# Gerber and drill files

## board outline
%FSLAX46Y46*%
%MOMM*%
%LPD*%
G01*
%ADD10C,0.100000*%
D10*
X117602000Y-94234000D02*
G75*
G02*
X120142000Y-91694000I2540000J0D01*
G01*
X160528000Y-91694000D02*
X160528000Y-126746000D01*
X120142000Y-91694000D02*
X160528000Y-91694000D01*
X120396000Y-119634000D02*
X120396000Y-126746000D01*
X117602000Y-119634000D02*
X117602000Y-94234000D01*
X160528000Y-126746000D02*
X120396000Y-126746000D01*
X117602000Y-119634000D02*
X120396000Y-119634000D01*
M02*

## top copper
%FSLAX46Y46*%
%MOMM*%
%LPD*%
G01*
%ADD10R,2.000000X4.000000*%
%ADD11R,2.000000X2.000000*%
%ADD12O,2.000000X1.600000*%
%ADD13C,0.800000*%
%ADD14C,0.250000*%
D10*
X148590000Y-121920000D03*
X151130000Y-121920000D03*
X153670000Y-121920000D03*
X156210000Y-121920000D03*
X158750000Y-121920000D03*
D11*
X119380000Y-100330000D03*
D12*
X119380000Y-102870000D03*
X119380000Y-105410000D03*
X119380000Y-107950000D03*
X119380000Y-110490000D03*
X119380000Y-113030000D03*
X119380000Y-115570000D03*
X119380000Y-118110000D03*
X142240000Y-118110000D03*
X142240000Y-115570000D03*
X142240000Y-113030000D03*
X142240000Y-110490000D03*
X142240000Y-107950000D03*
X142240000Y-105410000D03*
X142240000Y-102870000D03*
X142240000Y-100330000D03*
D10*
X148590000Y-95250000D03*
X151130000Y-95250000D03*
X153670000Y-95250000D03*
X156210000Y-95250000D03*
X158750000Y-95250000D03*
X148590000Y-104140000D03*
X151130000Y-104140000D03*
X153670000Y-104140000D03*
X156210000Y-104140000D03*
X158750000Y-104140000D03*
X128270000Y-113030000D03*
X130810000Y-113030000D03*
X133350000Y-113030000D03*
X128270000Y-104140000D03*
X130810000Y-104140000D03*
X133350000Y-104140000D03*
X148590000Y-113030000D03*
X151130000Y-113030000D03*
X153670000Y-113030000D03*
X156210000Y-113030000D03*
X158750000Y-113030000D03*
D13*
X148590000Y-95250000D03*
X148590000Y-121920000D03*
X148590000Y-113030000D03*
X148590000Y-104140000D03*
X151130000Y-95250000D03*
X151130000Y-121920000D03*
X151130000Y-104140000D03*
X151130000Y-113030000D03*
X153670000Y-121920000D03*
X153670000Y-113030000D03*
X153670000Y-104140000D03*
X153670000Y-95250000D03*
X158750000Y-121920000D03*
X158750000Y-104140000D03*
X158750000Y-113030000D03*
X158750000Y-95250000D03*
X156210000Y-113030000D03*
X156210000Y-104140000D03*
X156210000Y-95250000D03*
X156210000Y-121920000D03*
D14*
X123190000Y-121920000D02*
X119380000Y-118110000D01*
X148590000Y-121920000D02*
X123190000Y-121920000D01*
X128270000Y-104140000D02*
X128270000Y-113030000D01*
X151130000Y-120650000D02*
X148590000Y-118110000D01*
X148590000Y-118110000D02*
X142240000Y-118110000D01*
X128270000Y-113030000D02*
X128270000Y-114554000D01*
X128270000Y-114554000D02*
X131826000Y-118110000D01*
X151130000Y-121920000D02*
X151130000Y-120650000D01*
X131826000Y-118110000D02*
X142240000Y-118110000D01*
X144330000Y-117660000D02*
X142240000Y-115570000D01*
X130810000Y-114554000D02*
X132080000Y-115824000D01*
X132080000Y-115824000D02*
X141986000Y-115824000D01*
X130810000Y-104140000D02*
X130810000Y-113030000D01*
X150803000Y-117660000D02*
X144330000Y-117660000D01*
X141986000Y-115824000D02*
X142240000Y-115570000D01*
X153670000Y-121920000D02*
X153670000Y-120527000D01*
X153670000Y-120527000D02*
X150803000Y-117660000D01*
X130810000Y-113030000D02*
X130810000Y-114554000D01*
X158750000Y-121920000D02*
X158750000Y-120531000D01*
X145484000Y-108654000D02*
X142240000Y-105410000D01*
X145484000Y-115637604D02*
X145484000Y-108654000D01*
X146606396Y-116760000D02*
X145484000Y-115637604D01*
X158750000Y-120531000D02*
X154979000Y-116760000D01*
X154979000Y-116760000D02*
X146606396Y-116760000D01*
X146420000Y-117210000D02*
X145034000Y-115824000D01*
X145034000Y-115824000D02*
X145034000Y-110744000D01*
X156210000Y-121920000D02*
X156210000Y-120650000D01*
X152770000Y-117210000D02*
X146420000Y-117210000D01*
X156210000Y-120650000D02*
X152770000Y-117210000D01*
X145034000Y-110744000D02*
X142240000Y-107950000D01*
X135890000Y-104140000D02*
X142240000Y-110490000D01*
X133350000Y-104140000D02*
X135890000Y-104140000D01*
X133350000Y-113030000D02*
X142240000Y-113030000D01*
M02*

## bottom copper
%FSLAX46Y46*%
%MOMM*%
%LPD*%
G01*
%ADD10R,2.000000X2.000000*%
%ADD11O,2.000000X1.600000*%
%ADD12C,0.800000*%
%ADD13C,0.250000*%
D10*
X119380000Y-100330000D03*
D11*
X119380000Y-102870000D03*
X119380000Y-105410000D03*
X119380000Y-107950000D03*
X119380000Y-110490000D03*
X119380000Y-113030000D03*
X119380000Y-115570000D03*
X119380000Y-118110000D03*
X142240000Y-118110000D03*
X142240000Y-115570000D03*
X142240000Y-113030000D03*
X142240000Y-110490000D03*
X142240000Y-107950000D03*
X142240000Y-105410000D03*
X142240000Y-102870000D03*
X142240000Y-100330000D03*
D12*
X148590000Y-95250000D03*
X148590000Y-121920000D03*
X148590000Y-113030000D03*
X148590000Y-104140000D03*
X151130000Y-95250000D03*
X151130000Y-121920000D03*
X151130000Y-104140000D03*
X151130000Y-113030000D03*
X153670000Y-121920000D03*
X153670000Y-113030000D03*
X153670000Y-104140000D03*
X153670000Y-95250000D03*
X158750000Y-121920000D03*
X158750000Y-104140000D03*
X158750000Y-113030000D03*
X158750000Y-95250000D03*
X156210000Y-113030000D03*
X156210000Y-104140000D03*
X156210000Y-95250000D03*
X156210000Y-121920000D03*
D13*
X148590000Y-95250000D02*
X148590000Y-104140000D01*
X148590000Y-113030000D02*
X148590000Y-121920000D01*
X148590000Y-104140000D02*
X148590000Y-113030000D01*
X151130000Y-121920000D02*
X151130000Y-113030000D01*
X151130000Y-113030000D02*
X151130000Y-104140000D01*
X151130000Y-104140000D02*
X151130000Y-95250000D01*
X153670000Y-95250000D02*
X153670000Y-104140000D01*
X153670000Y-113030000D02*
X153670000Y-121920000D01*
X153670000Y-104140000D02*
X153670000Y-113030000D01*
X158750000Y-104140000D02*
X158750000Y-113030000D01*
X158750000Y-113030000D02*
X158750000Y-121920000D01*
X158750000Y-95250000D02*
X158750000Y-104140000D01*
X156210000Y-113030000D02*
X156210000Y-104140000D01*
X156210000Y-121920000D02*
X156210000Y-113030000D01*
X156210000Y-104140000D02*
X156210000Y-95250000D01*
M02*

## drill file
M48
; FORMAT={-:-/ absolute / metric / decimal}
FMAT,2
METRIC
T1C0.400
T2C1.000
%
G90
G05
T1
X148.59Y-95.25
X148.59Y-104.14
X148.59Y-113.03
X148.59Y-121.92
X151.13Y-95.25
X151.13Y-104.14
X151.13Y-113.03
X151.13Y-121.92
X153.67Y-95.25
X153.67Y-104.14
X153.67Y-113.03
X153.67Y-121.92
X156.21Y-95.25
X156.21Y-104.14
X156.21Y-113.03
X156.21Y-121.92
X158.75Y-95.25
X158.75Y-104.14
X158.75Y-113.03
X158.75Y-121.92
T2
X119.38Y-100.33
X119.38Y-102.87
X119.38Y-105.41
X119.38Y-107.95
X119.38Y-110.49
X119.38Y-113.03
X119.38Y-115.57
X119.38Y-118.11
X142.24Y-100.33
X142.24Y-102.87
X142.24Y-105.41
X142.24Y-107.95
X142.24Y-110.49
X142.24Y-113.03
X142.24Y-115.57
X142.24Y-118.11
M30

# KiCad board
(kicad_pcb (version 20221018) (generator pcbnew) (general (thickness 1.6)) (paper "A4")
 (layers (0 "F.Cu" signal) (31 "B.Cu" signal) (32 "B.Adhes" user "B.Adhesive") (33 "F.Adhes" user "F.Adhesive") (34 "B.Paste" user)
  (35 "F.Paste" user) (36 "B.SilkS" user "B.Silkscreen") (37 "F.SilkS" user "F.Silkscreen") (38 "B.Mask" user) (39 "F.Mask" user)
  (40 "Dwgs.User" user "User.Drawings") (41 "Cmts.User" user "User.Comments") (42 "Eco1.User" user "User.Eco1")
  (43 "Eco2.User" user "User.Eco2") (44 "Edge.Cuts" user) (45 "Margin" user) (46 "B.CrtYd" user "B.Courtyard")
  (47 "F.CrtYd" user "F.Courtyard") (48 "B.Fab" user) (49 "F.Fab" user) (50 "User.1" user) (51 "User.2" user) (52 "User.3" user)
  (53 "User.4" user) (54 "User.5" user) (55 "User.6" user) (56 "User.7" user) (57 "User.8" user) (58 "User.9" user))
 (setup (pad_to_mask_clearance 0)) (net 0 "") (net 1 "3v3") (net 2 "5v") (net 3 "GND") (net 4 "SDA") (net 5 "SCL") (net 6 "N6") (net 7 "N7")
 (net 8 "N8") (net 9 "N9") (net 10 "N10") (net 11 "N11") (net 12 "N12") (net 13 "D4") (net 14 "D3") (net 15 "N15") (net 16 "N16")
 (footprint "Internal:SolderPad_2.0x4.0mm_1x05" (layer "F.Cu") (at 153.67 124.46)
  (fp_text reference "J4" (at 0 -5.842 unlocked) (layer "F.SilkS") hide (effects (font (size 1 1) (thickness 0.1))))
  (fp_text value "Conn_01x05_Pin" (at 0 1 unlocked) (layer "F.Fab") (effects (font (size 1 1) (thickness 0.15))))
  (pad "1" smd rect (at -5.08 -2.54) (size 2 4) (layers "F.Cu" "F.Paste" "F.Mask") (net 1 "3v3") (thermal_bridge_angle 45))
  (pad "2" smd rect (at -2.54 -2.54) (size 2 4) (layers "F.Cu" "F.Paste" "F.Mask") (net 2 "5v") (thermal_bridge_angle 45))
  (pad "3" smd rect (at 0 -2.54) (size 2 4) (layers "F.Cu" "F.Paste" "F.Mask") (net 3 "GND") (thermal_bridge_angle 45))
  (pad "4" smd rect (at 2.54 -2.54) (size 2 4) (layers "F.Cu" "F.Paste" "F.Mask") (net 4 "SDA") (thermal_bridge_angle 45))
  (pad "5" smd rect (at 5.08 -2.54) (size 2 4) (layers "F.Cu" "F.Paste" "F.Mask") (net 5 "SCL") (thermal_bridge_angle 45)))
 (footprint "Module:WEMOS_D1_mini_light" (layer "F.Cu") (at 119.38 100.33)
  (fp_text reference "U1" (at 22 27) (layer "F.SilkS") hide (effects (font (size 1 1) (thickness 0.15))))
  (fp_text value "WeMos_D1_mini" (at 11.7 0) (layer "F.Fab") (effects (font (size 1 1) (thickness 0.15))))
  (pad "1" thru_hole rect (at 0 0) (size 2 2) (drill 1) (layers "*.Cu" "*.Mask") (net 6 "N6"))
  (pad "2" thru_hole oval (at 0 2.54) (size 2 1.6) (drill 1) (layers "*.Cu" "*.Mask") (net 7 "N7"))
  (pad "3" thru_hole oval (at 0 5.08) (size 2 1.6) (drill 1) (layers "*.Cu" "*.Mask") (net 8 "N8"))
  (pad "4" thru_hole oval (at 0 7.62) (size 2 1.6) (drill 1) (layers "*.Cu" "*.Mask") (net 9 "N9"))
  (pad "5" thru_hole oval (at 0 10.16) (size 2 1.6) (drill 1) (layers "*.Cu" "*.Mask") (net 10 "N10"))
  (pad "6" thru_hole oval (at 0 12.7) (size 2 1.6) (drill 1) (layers "*.Cu" "*.Mask") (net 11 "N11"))
  (pad "7" thru_hole oval (at 0 15.24) (size 2 1.6) (drill 1) (layers "*.Cu" "*.Mask") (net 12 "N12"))
  (pad "8" thru_hole oval (at 0 17.78) (size 2 1.6) (drill 1) (layers "*.Cu" "*.Mask") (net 1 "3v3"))
  (pad "9" thru_hole oval (at 22.86 17.78) (size 2 1.6) (drill 1) (layers "*.Cu" "*.Mask") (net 2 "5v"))
  (pad "10" thru_hole oval (at 22.86 15.24) (size 2 1.6) (drill 1) (layers "*.Cu" "*.Mask") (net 3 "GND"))
  (pad "11" thru_hole oval (at 22.86 12.7) (size 2 1.6) (drill 1) (layers "*.Cu" "*.Mask") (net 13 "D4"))
  (pad "12" thru_hole oval (at 22.86 10.16) (size 2 1.6) (drill 1) (layers "*.Cu" "*.Mask") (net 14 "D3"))
  (pad "13" thru_hole oval (at 22.86 7.62) (size 2 1.6) (drill 1) (layers "*.Cu" "*.Mask") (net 4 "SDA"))
  (pad "14" thru_hole oval (at 22.86 5.08) (size 2 1.6) (drill 1) (layers "*.Cu" "*.Mask") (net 5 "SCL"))
  (pad "15" thru_hole oval (at 22.86 2.54) (size 2 1.6) (drill 1) (layers "*.Cu" "*.Mask") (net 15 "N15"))
  (pad "16" thru_hole oval (at 22.86 0) (size 2 1.6) (drill 1) (layers "*.Cu" "*.Mask") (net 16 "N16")))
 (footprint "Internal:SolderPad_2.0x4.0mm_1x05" (layer "F.Cu") (at 153.67 97.79)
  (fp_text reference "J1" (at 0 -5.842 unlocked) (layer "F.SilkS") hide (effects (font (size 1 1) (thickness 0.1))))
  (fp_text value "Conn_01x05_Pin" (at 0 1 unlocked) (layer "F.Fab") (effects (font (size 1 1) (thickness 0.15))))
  (pad "1" smd rect (at -5.08 -2.54) (size 2 4) (layers "F.Cu" "F.Paste" "F.Mask") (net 1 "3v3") (thermal_bridge_angle 45))
  (pad "2" smd rect (at -2.54 -2.54) (size 2 4) (layers "F.Cu" "F.Paste" "F.Mask") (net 2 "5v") (thermal_bridge_angle 45))
  (pad "3" smd rect (at 0 -2.54) (size 2 4) (layers "F.Cu" "F.Paste" "F.Mask") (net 3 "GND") (thermal_bridge_angle 45))
  (pad "4" smd rect (at 2.54 -2.54) (size 2 4) (layers "F.Cu" "F.Paste" "F.Mask") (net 4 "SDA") (thermal_bridge_angle 45))
  (pad "5" smd rect (at 5.08 -2.54) (size 2 4) (layers "F.Cu" "F.Paste" "F.Mask") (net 5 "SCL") (thermal_bridge_angle 45)))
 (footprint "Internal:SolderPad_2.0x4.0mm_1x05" (layer "F.Cu") (at 153.67 106.68)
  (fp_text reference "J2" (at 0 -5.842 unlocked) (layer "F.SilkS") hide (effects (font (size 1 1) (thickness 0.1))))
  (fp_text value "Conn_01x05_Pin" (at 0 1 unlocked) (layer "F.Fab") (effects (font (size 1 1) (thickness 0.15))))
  (pad "1" smd rect (at -5.08 -2.54) (size 2 4) (layers "F.Cu" "F.Paste" "F.Mask") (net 1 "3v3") (thermal_bridge_angle 45))
  (pad "2" smd rect (at -2.54 -2.54) (size 2 4) (layers "F.Cu" "F.Paste" "F.Mask") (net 2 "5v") (thermal_bridge_angle 45))
  (pad "3" smd rect (at 0 -2.54) (size 2 4) (layers "F.Cu" "F.Paste" "F.Mask") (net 3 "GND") (thermal_bridge_angle 45))
  (pad "4" smd rect (at 2.54 -2.54) (size 2 4) (layers "F.Cu" "F.Paste" "F.Mask") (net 4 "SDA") (thermal_bridge_angle 45))
  (pad "5" smd rect (at 5.08 -2.54) (size 2 4) (layers "F.Cu" "F.Paste" "F.Mask") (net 5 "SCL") (thermal_bridge_angle 45)))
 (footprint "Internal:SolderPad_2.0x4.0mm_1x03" (layer "F.Cu") (at 130.81 115.57)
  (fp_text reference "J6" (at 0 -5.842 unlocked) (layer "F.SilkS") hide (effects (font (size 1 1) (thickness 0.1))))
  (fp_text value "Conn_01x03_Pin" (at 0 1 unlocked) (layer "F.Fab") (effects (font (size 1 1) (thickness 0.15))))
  (pad "1" smd rect (at -2.54 -2.54) (size 2 4) (layers "F.Cu" "F.Paste" "F.Mask") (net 2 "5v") (thermal_bridge_angle 45))
  (pad "2" smd rect (at 0 -2.54) (size 2 4) (layers "F.Cu" "F.Paste" "F.Mask") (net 3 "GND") (thermal_bridge_angle 45))
  (pad "3" smd rect (at 2.54 -2.54) (size 2 4) (layers "F.Cu" "F.Paste" "F.Mask") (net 13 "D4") (thermal_bridge_angle 45)))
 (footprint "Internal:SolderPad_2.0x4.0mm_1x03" (layer "F.Cu") (at 130.81 106.68)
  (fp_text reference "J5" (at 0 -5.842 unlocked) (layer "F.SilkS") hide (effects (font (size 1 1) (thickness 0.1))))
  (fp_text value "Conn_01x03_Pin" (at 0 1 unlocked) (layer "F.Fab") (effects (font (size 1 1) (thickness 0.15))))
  (pad "1" smd rect (at -2.54 -2.54) (size 2 4) (layers "F.Cu" "F.Paste" "F.Mask") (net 2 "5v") (thermal_bridge_angle 45))
  (pad "2" smd rect (at 0 -2.54) (size 2 4) (layers "F.Cu" "F.Paste" "F.Mask") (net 3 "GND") (thermal_bridge_angle 45))
  (pad "3" smd rect (at 2.54 -2.54) (size 2 4) (layers "F.Cu" "F.Paste" "F.Mask") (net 14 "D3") (thermal_bridge_angle 45)))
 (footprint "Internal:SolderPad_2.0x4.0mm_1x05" (layer "F.Cu") (at 153.67 115.57)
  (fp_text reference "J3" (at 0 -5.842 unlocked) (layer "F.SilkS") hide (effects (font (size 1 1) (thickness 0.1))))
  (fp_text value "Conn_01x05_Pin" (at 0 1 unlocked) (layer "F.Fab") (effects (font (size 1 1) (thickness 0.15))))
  (pad "1" smd rect (at -5.08 -2.54) (size 2 4) (layers "F.Cu" "F.Paste" "F.Mask") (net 1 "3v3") (thermal_bridge_angle 45))
  (pad "2" smd rect (at -2.54 -2.54) (size 2 4) (layers "F.Cu" "F.Paste" "F.Mask") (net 2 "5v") (thermal_bridge_angle 45))
  (pad "3" smd rect (at 0 -2.54) (size 2 4) (layers "F.Cu" "F.Paste" "F.Mask") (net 3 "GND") (thermal_bridge_angle 45))
  (pad "4" smd rect (at 2.54 -2.54) (size 2 4) (layers "F.Cu" "F.Paste" "F.Mask") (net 4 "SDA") (thermal_bridge_angle 45))
  (pad "5" smd rect (at 5.08 -2.54) (size 2 4) (layers "F.Cu" "F.Paste" "F.Mask") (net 5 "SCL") (thermal_bridge_angle 45)))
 (gr_arc (start 117.602 94.234) (mid 118.345949 92.437949) (end 120.142 91.694) (stroke (width 0.1) (type default)) (layer "Edge.Cuts"))
 (gr_line (start 160.528 91.694) (end 160.528 126.746) (stroke (width 0.1) (type default)) (layer "Edge.Cuts"))
 (gr_line (start 120.142 91.694) (end 160.528 91.694) (stroke (width 0.1) (type default)) (layer "Edge.Cuts"))
 (gr_line (start 120.396 119.634) (end 120.396 126.746) (stroke (width 0.1) (type default)) (layer "Edge.Cuts"))
 (gr_line (start 117.602 119.634) (end 117.602 94.234) (stroke (width 0.1) (type default)) (layer "Edge.Cuts"))
 (gr_line (start 160.528 126.746) (end 120.396 126.746) (stroke (width 0.1) (type default)) (layer "Edge.Cuts"))
 (gr_line (start 117.602 119.634) (end 120.396 119.634) (stroke (width 0.1) (type default)) (layer "Edge.Cuts"))
 (segment (start 123.19 121.92) (end 119.38 118.11) (width 0.25) (layer "F.Cu") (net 1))
 (segment (start 148.59 121.92) (end 123.19 121.92) (width 0.25) (layer "F.Cu") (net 1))
 (via (at 148.59 95.25) (size 0.8) (drill 0.4) (layers "F.Cu" "B.Cu") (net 1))
 (via (at 148.59 121.92) (size 0.8) (drill 0.4) (layers "F.Cu" "B.Cu") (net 1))
 (via (at 148.59 113.03) (size 0.8) (drill 0.4) (layers "F.Cu" "B.Cu") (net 1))
 (via (at 148.59 104.14) (size 0.8) (drill 0.4) (layers "F.Cu" "B.Cu") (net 1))
 (segment (start 148.59 95.25) (end 148.59 104.14) (width 0.25) (layer "B.Cu") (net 1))
 (segment (start 148.59 113.03) (end 148.59 121.92) (width 0.25) (layer "B.Cu") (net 1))
 (segment (start 148.59 104.14) (end 148.59 113.03) (width 0.25) (layer "B.Cu") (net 1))
 (segment (start 128.27 104.14) (end 128.27 113.03) (width 0.25) (layer "F.Cu") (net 2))
 (segment (start 151.13 120.65) (end 148.59 118.11) (width 0.25) (layer "F.Cu") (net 2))
 (segment (start 148.59 118.11) (end 142.24 118.11) (width 0.25) (layer "F.Cu") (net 2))
 (segment (start 128.27 113.03) (end 128.27 114.554) (width 0.25) (layer "F.Cu") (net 2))
 (segment (start 128.27 114.554) (end 131.826 118.11) (width 0.25) (layer "F.Cu") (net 2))
 (segment (start 151.13 121.92) (end 151.13 120.65) (width 0.25) (layer "F.Cu") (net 2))
 (segment (start 131.826 118.11) (end 142.24 118.11) (width 0.25) (layer "F.Cu") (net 2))
 (via (at 151.13 95.25) (size 0.8) (drill 0.4) (layers "F.Cu" "B.Cu") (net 2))
 (via (at 151.13 121.92) (size 0.8) (drill 0.4) (layers "F.Cu" "B.Cu") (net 2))
 (via (at 151.13 104.14) (size 0.8) (drill 0.4) (layers "F.Cu" "B.Cu") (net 2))
 (via (at 151.13 113.03) (size 0.8) (drill 0.4) (layers "F.Cu" "B.Cu") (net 2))
 (segment (start 151.13 121.92) (end 151.13 113.03) (width 0.25) (layer "B.Cu") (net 2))
 (segment (start 151.13 113.03) (end 151.13 104.14) (width 0.25) (layer "B.Cu") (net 2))
 (segment (start 151.13 104.14) (end 151.13 95.25) (width 0.25) (layer "B.Cu") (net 2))
 (segment (start 144.33 117.66) (end 142.24 115.57) (width 0.25) (layer "F.Cu") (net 3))
 (segment (start 130.81 114.554) (end 132.08 115.824) (width 0.25) (layer "F.Cu") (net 3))
 (segment (start 132.08 115.824) (end 141.986 115.824) (width 0.25) (layer "F.Cu") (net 3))
 (segment (start 130.81 104.14) (end 130.81 113.03) (width 0.25) (layer "F.Cu") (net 3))
 (segment (start 150.803 117.66) (end 144.33 117.66) (width 0.25) (layer "F.Cu") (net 3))
 (segment (start 141.986 115.824) (end 142.24 115.57) (width 0.25) (layer "F.Cu") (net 3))
 (segment (start 153.67 121.92) (end 153.67 120.527) (width 0.25) (layer "F.Cu") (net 3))
 (segment (start 153.67 120.527) (end 150.803 117.66) (width 0.25) (layer "F.Cu") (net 3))
 (segment (start 130.81 113.03) (end 130.81 114.554) (width 0.25) (layer "F.Cu") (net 3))
 (via (at 153.67 121.92) (size 0.8) (drill 0.4) (layers "F.Cu" "B.Cu") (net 3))
 (via (at 153.67 113.03) (size 0.8) (drill 0.4) (layers "F.Cu" "B.Cu") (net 3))
 (via (at 153.67 104.14) (size 0.8) (drill 0.4) (layers "F.Cu" "B.Cu") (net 3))
 (via (at 153.67 95.25) (size 0.8) (drill 0.4) (layers "F.Cu" "B.Cu") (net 3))
 (segment (start 153.67 95.25) (end 153.67 104.14) (width 0.25) (layer "B.Cu") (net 3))
 (segment (start 153.67 113.03) (end 153.67 121.92) (width 0.25) (layer "B.Cu") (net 3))
 (segment (start 153.67 104.14) (end 153.67 113.03) (width 0.25) (layer "B.Cu") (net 3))
 (segment (start 158.75 121.92) (end 158.75 120.531) (width 0.25) (layer "F.Cu") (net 5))
 (segment (start 145.484 108.654) (end 142.24 105.41) (width 0.25) (layer "F.Cu") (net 5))
 (segment (start 145.484 115.637604) (end 145.484 108.654) (width 0.25) (layer "F.Cu") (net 5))
 (segment (start 146.606396 116.76) (end 145.484 115.637604) (width 0.25) (layer "F.Cu") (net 5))
 (segment (start 158.75 120.531) (end 154.979 116.76) (width 0.25) (layer "F.Cu") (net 5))
 (segment (start 154.979 116.76) (end 146.606396 116.76) (width 0.25) (layer "F.Cu") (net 5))
 (via (at 158.75 121.92) (size 0.8) (drill 0.4) (layers "F.Cu" "B.Cu") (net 5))
 (via (at 158.75 104.14) (size 0.8) (drill 0.4) (layers "F.Cu" "B.Cu") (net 5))
 (via (at 158.75 113.03) (size 0.8) (drill 0.4) (layers "F.Cu" "B.Cu") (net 5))
 (via (at 158.75 95.25) (size 0.8) (drill 0.4) (layers "F.Cu" "B.Cu") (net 5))
 (segment (start 158.75 104.14) (end 158.75 113.03) (width 0.25) (layer "B.Cu") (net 5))
 (segment (start 158.75 113.03) (end 158.75 121.92) (width 0.25) (layer "B.Cu") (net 5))
 (segment (start 158.75 95.25) (end 158.75 104.14) (width 0.25) (layer "B.Cu") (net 5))
 (segment (start 146.42 117.21) (end 145.034 115.824) (width 0.25) (layer "F.Cu") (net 4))
 (segment (start 145.034 115.824) (end 145.034 110.744) (width 0.25) (layer "F.Cu") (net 4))
 (segment (start 156.21 121.92) (end 156.21 120.65) (width 0.25) (layer "F.Cu") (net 4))
 (segment (start 152.77 117.21) (end 146.42 117.21) (width 0.25) (layer "F.Cu") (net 4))
 (segment (start 156.21 120.65) (end 152.77 117.21) (width 0.25) (layer "F.Cu") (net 4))
 (segment (start 145.034 110.744) (end 142.24 107.95) (width 0.25) (layer "F.Cu") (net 4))
 (via (at 156.21 113.03) (size 0.8) (drill 0.4) (layers "F.Cu" "B.Cu") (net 4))
 (via (at 156.21 104.14) (size 0.8) (drill 0.4) (layers "F.Cu" "B.Cu") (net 4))
 (via (at 156.21 95.25) (size 0.8) (drill 0.4) (layers "F.Cu" "B.Cu") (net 4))
 (via (at 156.21 121.92) (size 0.8) (drill 0.4) (layers "F.Cu" "B.Cu") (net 4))
 (segment (start 156.21 113.03) (end 156.21 104.14) (width 0.25) (layer "B.Cu") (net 4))
 (segment (start 156.21 121.92) (end 156.21 113.03) (width 0.25) (layer "B.Cu") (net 4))
 (segment (start 156.21 104.14) (end 156.21 95.25) (width 0.25) (layer "B.Cu") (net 4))
 (segment (start 135.89 104.14) (end 142.24 110.49) (width 0.25) (layer "F.Cu") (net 14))
 (segment (start 133.35 104.14) (end 135.89 104.14) (width 0.25) (layer "F.Cu") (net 14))
 (segment (start 133.35 113.03) (end 142.24 113.03) (width 0.25) (layer "F.Cu") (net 13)))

